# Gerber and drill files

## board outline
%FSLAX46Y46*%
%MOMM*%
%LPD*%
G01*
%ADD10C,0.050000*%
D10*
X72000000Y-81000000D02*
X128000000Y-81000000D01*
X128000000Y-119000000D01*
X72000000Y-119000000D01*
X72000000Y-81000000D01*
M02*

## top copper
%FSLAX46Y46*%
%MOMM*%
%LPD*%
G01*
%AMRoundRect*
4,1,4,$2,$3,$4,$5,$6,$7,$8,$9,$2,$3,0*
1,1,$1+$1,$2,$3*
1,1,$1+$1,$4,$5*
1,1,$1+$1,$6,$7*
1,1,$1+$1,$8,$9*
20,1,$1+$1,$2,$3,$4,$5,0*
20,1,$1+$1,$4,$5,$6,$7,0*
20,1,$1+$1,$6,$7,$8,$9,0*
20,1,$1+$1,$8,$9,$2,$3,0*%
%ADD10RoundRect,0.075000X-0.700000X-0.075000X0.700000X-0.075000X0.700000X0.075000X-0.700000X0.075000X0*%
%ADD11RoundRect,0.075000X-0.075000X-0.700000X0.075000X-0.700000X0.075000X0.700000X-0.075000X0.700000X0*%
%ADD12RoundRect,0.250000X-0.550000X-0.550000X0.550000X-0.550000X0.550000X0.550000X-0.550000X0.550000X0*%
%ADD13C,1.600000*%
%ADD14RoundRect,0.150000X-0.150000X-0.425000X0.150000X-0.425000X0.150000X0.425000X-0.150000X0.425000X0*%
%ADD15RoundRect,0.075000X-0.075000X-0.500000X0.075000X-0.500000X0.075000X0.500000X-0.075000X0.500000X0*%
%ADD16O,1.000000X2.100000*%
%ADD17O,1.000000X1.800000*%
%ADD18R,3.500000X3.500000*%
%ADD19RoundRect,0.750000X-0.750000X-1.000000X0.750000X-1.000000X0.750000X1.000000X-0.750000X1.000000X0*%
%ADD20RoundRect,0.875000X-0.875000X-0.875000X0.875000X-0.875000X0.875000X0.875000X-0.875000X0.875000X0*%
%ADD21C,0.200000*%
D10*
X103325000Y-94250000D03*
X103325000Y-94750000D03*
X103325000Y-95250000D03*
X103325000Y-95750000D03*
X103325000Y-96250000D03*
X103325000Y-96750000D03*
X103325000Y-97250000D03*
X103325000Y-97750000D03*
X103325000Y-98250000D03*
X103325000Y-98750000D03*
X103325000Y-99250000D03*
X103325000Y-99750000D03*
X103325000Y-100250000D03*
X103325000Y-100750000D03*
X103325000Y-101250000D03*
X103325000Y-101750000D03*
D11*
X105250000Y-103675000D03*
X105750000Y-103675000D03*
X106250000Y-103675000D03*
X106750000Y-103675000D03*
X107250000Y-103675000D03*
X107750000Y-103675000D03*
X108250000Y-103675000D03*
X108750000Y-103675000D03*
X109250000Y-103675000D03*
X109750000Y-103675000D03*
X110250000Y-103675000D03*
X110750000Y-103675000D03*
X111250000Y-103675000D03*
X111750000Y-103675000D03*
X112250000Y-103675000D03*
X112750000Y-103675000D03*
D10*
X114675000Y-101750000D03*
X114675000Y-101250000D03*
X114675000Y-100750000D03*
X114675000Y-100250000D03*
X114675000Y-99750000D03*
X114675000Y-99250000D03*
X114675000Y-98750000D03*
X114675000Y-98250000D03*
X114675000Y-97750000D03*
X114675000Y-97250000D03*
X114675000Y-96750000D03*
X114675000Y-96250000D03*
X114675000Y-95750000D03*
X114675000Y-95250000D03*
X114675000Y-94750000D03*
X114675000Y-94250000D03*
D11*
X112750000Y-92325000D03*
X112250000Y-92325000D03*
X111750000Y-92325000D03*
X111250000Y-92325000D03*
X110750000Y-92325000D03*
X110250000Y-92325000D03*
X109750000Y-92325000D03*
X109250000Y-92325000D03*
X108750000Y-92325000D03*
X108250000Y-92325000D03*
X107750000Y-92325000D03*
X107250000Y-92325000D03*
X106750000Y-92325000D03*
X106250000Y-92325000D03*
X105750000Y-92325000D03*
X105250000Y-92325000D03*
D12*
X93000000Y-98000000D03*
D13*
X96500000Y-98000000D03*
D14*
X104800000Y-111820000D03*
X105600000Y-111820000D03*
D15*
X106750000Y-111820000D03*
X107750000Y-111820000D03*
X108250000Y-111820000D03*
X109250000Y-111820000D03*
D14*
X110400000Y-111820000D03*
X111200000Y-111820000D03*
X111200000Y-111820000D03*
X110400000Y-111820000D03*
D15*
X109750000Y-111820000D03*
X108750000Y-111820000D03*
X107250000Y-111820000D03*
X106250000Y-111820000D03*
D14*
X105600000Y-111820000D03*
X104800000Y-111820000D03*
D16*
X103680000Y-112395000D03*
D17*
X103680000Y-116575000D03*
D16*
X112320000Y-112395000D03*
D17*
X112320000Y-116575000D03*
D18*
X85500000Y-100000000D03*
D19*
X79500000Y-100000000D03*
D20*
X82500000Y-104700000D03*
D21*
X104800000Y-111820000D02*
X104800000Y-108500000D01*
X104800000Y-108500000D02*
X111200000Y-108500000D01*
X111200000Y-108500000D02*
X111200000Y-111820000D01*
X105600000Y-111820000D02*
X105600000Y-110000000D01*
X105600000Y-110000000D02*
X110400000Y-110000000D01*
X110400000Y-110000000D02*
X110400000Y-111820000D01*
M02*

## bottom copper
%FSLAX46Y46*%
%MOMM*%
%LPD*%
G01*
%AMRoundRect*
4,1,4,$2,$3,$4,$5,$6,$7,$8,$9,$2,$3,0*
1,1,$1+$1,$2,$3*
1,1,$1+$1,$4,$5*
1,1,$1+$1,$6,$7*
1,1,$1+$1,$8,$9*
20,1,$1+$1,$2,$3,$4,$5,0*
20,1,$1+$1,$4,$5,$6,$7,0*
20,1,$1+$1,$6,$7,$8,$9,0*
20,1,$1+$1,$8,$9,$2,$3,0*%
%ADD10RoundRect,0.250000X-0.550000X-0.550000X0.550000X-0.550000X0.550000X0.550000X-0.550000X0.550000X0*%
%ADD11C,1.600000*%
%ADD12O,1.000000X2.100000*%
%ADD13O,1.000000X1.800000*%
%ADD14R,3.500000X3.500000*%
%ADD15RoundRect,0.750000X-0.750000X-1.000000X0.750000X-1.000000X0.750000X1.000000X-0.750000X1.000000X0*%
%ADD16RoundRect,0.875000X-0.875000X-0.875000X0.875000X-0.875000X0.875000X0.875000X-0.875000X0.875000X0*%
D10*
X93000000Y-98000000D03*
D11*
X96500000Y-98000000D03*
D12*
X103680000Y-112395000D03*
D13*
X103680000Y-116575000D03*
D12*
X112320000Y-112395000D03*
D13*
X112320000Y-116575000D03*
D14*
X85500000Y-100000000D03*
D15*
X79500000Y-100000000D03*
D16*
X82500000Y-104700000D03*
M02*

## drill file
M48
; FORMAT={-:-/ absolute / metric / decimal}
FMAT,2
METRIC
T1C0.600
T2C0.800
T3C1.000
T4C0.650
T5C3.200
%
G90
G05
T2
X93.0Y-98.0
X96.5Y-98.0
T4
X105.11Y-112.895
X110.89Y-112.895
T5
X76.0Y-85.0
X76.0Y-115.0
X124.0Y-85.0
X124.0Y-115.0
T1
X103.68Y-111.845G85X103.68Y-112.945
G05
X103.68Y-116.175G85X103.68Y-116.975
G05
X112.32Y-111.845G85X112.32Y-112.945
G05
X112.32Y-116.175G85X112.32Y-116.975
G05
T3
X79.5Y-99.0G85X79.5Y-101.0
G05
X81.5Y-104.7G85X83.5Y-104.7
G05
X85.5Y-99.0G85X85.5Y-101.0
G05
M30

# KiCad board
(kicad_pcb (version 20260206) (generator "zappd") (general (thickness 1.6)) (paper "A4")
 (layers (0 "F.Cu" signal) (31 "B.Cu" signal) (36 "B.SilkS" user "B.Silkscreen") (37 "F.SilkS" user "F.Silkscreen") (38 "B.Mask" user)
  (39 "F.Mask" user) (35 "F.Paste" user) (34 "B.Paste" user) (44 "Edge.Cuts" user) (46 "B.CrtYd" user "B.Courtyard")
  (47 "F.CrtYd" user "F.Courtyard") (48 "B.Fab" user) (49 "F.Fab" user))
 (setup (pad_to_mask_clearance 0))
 (gr_rect (start 72.0 81.0) (end 128.0 119.0) (stroke (width 0.05) (type default)) (fill none) (layer "Edge.Cuts"))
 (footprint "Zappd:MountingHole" (layer "F.Cu") (at 76.0 85.0)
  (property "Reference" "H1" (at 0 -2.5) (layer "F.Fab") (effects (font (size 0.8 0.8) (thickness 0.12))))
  (pad "" np_thru_hole circle (at 0 0) (size 3.2 3.2) (drill 3.2) (layers "*.Cu" "*.Mask")))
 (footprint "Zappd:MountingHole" (layer "F.Cu") (at 124.0 85.0)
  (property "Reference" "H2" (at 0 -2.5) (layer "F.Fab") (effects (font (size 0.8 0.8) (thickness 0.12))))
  (pad "" np_thru_hole circle (at 0 0) (size 3.2 3.2) (drill 3.2) (layers "*.Cu" "*.Mask")))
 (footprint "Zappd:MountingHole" (layer "F.Cu") (at 124.0 115.0)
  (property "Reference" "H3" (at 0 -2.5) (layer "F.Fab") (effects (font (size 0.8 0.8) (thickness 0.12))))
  (pad "" np_thru_hole circle (at 0 0) (size 3.2 3.2) (drill 3.2) (layers "*.Cu" "*.Mask")))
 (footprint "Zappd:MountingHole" (layer "F.Cu") (at 76.0 115.0)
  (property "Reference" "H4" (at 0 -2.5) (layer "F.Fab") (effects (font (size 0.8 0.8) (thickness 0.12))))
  (pad "" np_thru_hole circle (at 0 0) (size 3.2 3.2) (drill 3.2) (layers "*.Cu" "*.Mask")))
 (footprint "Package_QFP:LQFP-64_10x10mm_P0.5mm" (layer "F.Cu") (at 109 98)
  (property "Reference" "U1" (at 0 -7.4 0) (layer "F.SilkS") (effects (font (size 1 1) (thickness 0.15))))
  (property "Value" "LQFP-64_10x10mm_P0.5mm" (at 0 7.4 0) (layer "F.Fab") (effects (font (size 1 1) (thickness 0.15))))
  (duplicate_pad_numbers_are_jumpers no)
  (pad "1" smd roundrect (at -5.675 -3.75) (size 1.55 0.3) (layers "F.Cu" "F.Mask" "F.Paste") (roundrect_rratio 0.25))
  (pad "2" smd roundrect (at -5.675 -3.25) (size 1.55 0.3) (layers "F.Cu" "F.Mask" "F.Paste") (roundrect_rratio 0.25))
  (pad "3" smd roundrect (at -5.675 -2.75) (size 1.55 0.3) (layers "F.Cu" "F.Mask" "F.Paste") (roundrect_rratio 0.25))
  (pad "4" smd roundrect (at -5.675 -2.25) (size 1.55 0.3) (layers "F.Cu" "F.Mask" "F.Paste") (roundrect_rratio 0.25))
  (pad "5" smd roundrect (at -5.675 -1.75) (size 1.55 0.3) (layers "F.Cu" "F.Mask" "F.Paste") (roundrect_rratio 0.25))
  (pad "6" smd roundrect (at -5.675 -1.25) (size 1.55 0.3) (layers "F.Cu" "F.Mask" "F.Paste") (roundrect_rratio 0.25))
  (pad "7" smd roundrect (at -5.675 -0.75) (size 1.55 0.3) (layers "F.Cu" "F.Mask" "F.Paste") (roundrect_rratio 0.25))
  (pad "8" smd roundrect (at -5.675 -0.25) (size 1.55 0.3) (layers "F.Cu" "F.Mask" "F.Paste") (roundrect_rratio 0.25))
  (pad "9" smd roundrect (at -5.675 0.25) (size 1.55 0.3) (layers "F.Cu" "F.Mask" "F.Paste") (roundrect_rratio 0.25))
  (pad "10" smd roundrect (at -5.675 0.75) (size 1.55 0.3) (layers "F.Cu" "F.Mask" "F.Paste") (roundrect_rratio 0.25))
  (pad "11" smd roundrect (at -5.675 1.25) (size 1.55 0.3) (layers "F.Cu" "F.Mask" "F.Paste") (roundrect_rratio 0.25))
  (pad "12" smd roundrect (at -5.675 1.75) (size 1.55 0.3) (layers "F.Cu" "F.Mask" "F.Paste") (roundrect_rratio 0.25))
  (pad "13" smd roundrect (at -5.675 2.25) (size 1.55 0.3) (layers "F.Cu" "F.Mask" "F.Paste") (roundrect_rratio 0.25))
  (pad "14" smd roundrect (at -5.675 2.75) (size 1.55 0.3) (layers "F.Cu" "F.Mask" "F.Paste") (roundrect_rratio 0.25))
  (pad "15" smd roundrect (at -5.675 3.25) (size 1.55 0.3) (layers "F.Cu" "F.Mask" "F.Paste") (roundrect_rratio 0.25))
  (pad "16" smd roundrect (at -5.675 3.75) (size 1.55 0.3) (layers "F.Cu" "F.Mask" "F.Paste") (roundrect_rratio 0.25))
  (pad "17" smd roundrect (at -3.75 5.675) (size 0.3 1.55) (layers "F.Cu" "F.Mask" "F.Paste") (roundrect_rratio 0.25))
  (pad "18" smd roundrect (at -3.25 5.675) (size 0.3 1.55) (layers "F.Cu" "F.Mask" "F.Paste") (roundrect_rratio 0.25))
  (pad "19" smd roundrect (at -2.75 5.675) (size 0.3 1.55) (layers "F.Cu" "F.Mask" "F.Paste") (roundrect_rratio 0.25))
  (pad "20" smd roundrect (at -2.25 5.675) (size 0.3 1.55) (layers "F.Cu" "F.Mask" "F.Paste") (roundrect_rratio 0.25))
  (pad "21" smd roundrect (at -1.75 5.675) (size 0.3 1.55) (layers "F.Cu" "F.Mask" "F.Paste") (roundrect_rratio 0.25))
  (pad "22" smd roundrect (at -1.25 5.675) (size 0.3 1.55) (layers "F.Cu" "F.Mask" "F.Paste") (roundrect_rratio 0.25))
  (pad "23" smd roundrect (at -0.75 5.675) (size 0.3 1.55) (layers "F.Cu" "F.Mask" "F.Paste") (roundrect_rratio 0.25))
  (pad "24" smd roundrect (at -0.25 5.675) (size 0.3 1.55) (layers "F.Cu" "F.Mask" "F.Paste") (roundrect_rratio 0.25))
  (pad "25" smd roundrect (at 0.25 5.675) (size 0.3 1.55) (layers "F.Cu" "F.Mask" "F.Paste") (roundrect_rratio 0.25))
  (pad "26" smd roundrect (at 0.75 5.675) (size 0.3 1.55) (layers "F.Cu" "F.Mask" "F.Paste") (roundrect_rratio 0.25))
  (pad "27" smd roundrect (at 1.25 5.675) (size 0.3 1.55) (layers "F.Cu" "F.Mask" "F.Paste") (roundrect_rratio 0.25))
  (pad "28" smd roundrect (at 1.75 5.675) (size 0.3 1.55) (layers "F.Cu" "F.Mask" "F.Paste") (roundrect_rratio 0.25))
  (pad "29" smd roundrect (at 2.25 5.675) (size 0.3 1.55) (layers "F.Cu" "F.Mask" "F.Paste") (roundrect_rratio 0.25))
  (pad "30" smd roundrect (at 2.75 5.675) (size 0.3 1.55) (layers "F.Cu" "F.Mask" "F.Paste") (roundrect_rratio 0.25))
  (pad "31" smd roundrect (at 3.25 5.675) (size 0.3 1.55) (layers "F.Cu" "F.Mask" "F.Paste") (roundrect_rratio 0.25))
  (pad "32" smd roundrect (at 3.75 5.675) (size 0.3 1.55) (layers "F.Cu" "F.Mask" "F.Paste") (roundrect_rratio 0.25))
  (pad "33" smd roundrect (at 5.675 3.75) (size 1.55 0.3) (layers "F.Cu" "F.Mask" "F.Paste") (roundrect_rratio 0.25))
  (pad "34" smd roundrect (at 5.675 3.25) (size 1.55 0.3) (layers "F.Cu" "F.Mask" "F.Paste") (roundrect_rratio 0.25))
  (pad "35" smd roundrect (at 5.675 2.75) (size 1.55 0.3) (layers "F.Cu" "F.Mask" "F.Paste") (roundrect_rratio 0.25))
  (pad "36" smd roundrect (at 5.675 2.25) (size 1.55 0.3) (layers "F.Cu" "F.Mask" "F.Paste") (roundrect_rratio 0.25))
  (pad "37" smd roundrect (at 5.675 1.75) (size 1.55 0.3) (layers "F.Cu" "F.Mask" "F.Paste") (roundrect_rratio 0.25))
  (pad "38" smd roundrect (at 5.675 1.25) (size 1.55 0.3) (layers "F.Cu" "F.Mask" "F.Paste") (roundrect_rratio 0.25))
  (pad "39" smd roundrect (at 5.675 0.75) (size 1.55 0.3) (layers "F.Cu" "F.Mask" "F.Paste") (roundrect_rratio 0.25))
  (pad "40" smd roundrect (at 5.675 0.25) (size 1.55 0.3) (layers "F.Cu" "F.Mask" "F.Paste") (roundrect_rratio 0.25))
  (pad "41" smd roundrect (at 5.675 -0.25) (size 1.55 0.3) (layers "F.Cu" "F.Mask" "F.Paste") (roundrect_rratio 0.25))
  (pad "42" smd roundrect (at 5.675 -0.75) (size 1.55 0.3) (layers "F.Cu" "F.Mask" "F.Paste") (roundrect_rratio 0.25))
  (pad "43" smd roundrect (at 5.675 -1.25) (size 1.55 0.3) (layers "F.Cu" "F.Mask" "F.Paste") (roundrect_rratio 0.25))
  (pad "44" smd roundrect (at 5.675 -1.75) (size 1.55 0.3) (layers "F.Cu" "F.Mask" "F.Paste") (roundrect_rratio 0.25))
  (pad "45" smd roundrect (at 5.675 -2.25) (size 1.55 0.3) (layers "F.Cu" "F.Mask" "F.Paste") (roundrect_rratio 0.25))
  (pad "46" smd roundrect (at 5.675 -2.75) (size 1.55 0.3) (layers "F.Cu" "F.Mask" "F.Paste") (roundrect_rratio 0.25))
  (pad "47" smd roundrect (at 5.675 -3.25) (size 1.55 0.3) (layers "F.Cu" "F.Mask" "F.Paste") (roundrect_rratio 0.25))
  (pad "48" smd roundrect (at 5.675 -3.75) (size 1.55 0.3) (layers "F.Cu" "F.Mask" "F.Paste") (roundrect_rratio 0.25))
  (pad "49" smd roundrect (at 3.75 -5.675) (size 0.3 1.55) (layers "F.Cu" "F.Mask" "F.Paste") (roundrect_rratio 0.25))
  (pad "50" smd roundrect (at 3.25 -5.675) (size 0.3 1.55) (layers "F.Cu" "F.Mask" "F.Paste") (roundrect_rratio 0.25))
  (pad "51" smd roundrect (at 2.75 -5.675) (size 0.3 1.55) (layers "F.Cu" "F.Mask" "F.Paste") (roundrect_rratio 0.25))
  (pad "52" smd roundrect (at 2.25 -5.675) (size 0.3 1.55) (layers "F.Cu" "F.Mask" "F.Paste") (roundrect_rratio 0.25))
  (pad "53" smd roundrect (at 1.75 -5.675) (size 0.3 1.55) (layers "F.Cu" "F.Mask" "F.Paste") (roundrect_rratio 0.25))
  (pad "54" smd roundrect (at 1.25 -5.675) (size 0.3 1.55) (layers "F.Cu" "F.Mask" "F.Paste") (roundrect_rratio 0.25))
  (pad "55" smd roundrect (at 0.75 -5.675) (size 0.3 1.55) (layers "F.Cu" "F.Mask" "F.Paste") (roundrect_rratio 0.25))
  (pad "56" smd roundrect (at 0.25 -5.675) (size 0.3 1.55) (layers "F.Cu" "F.Mask" "F.Paste") (roundrect_rratio 0.25))
  (pad "57" smd roundrect (at -0.25 -5.675) (size 0.3 1.55) (layers "F.Cu" "F.Mask" "F.Paste") (roundrect_rratio 0.25))
  (pad "58" smd roundrect (at -0.75 -5.675) (size 0.3 1.55) (layers "F.Cu" "F.Mask" "F.Paste") (roundrect_rratio 0.25))
  (pad "59" smd roundrect (at -1.25 -5.675) (size 0.3 1.55) (layers "F.Cu" "F.Mask" "F.Paste") (roundrect_rratio 0.25))
  (pad "60" smd roundrect (at -1.75 -5.675) (size 0.3 1.55) (layers "F.Cu" "F.Mask" "F.Paste") (roundrect_rratio 0.25))
  (pad "61" smd roundrect (at -2.25 -5.675) (size 0.3 1.55) (layers "F.Cu" "F.Mask" "F.Paste") (roundrect_rratio 0.25))
  (pad "62" smd roundrect (at -2.75 -5.675) (size 0.3 1.55) (layers "F.Cu" "F.Mask" "F.Paste") (roundrect_rratio 0.25))
  (pad "63" smd roundrect (at -3.25 -5.675) (size 0.3 1.55) (layers "F.Cu" "F.Mask" "F.Paste") (roundrect_rratio 0.25))
  (pad "64" smd roundrect (at -3.75 -5.675) (size 0.3 1.55) (layers "F.Cu" "F.Mask" "F.Paste") (roundrect_rratio 0.25)))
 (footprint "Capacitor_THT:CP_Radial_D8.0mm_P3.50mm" (layer "F.Cu") (at 93 98)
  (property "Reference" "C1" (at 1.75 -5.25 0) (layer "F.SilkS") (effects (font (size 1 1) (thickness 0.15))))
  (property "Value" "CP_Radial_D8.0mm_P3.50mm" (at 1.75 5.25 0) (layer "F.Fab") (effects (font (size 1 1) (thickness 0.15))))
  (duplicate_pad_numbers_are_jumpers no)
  (pad "1" thru_hole roundrect (at 0 0) (size 1.6 1.6) (drill 0.8) (layers "*.Cu" "*.Mask") (remove_unused_layers no)
   (roundrect_rratio 0.15625))
  (pad "2" thru_hole circle (at 3.5 0) (size 1.6 1.6) (drill 0.8) (layers "*.Cu" "*.Mask") (remove_unused_layers no)))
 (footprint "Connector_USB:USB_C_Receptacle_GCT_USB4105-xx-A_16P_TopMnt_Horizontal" (layer "F.Cu") (at 108 115.5)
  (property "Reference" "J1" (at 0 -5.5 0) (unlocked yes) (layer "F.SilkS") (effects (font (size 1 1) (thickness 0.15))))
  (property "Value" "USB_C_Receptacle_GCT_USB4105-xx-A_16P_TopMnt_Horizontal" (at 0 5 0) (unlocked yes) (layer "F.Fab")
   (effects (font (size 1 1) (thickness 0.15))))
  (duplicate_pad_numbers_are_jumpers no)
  (pad "" np_thru_hole circle (at -2.89 -2.605) (size 0.65 0.65) (drill 0.65) (layers "*.Cu" "*.Mask"))
  (pad "" np_thru_hole circle (at 2.89 -2.605) (size 0.65 0.65) (drill 0.65) (layers "*.Cu" "*.Mask"))
  (pad "A1" smd roundrect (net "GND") (at -3.2 -3.68) (size 0.6 1.15) (layers "F.Cu" "F.Mask" "F.Paste") (roundrect_rratio 0.25))
  (pad "A4" smd roundrect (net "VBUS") (at -2.4 -3.68) (size 0.6 1.15) (layers "F.Cu" "F.Mask" "F.Paste") (roundrect_rratio 0.25))
  (pad "A5" smd roundrect (at -1.25 -3.68) (size 0.3 1.15) (layers "F.Cu" "F.Mask" "F.Paste") (roundrect_rratio 0.25))
  (pad "A6" smd roundrect (at -0.25 -3.68) (size 0.3 1.15) (layers "F.Cu" "F.Mask" "F.Paste") (roundrect_rratio 0.25))
  (pad "A7" smd roundrect (at 0.25 -3.68) (size 0.3 1.15) (layers "F.Cu" "F.Mask" "F.Paste") (roundrect_rratio 0.25))
  (pad "A8" smd roundrect (at 1.25 -3.68) (size 0.3 1.15) (layers "F.Cu" "F.Mask" "F.Paste") (roundrect_rratio 0.25))
  (pad "A9" smd roundrect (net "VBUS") (at 2.4 -3.68) (size 0.6 1.15) (layers "F.Cu" "F.Mask" "F.Paste") (roundrect_rratio 0.25))
  (pad "A12" smd roundrect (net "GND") (at 3.2 -3.68) (size 0.6 1.15) (layers "F.Cu" "F.Mask" "F.Paste") (roundrect_rratio 0.25))
  (pad "B1" smd roundrect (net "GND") (at 3.2 -3.68) (size 0.6 1.15) (layers "F.Cu" "F.Mask" "F.Paste") (roundrect_rratio 0.25))
  (pad "B4" smd roundrect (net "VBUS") (at 2.4 -3.68) (size 0.6 1.15) (layers "F.Cu" "F.Mask" "F.Paste") (roundrect_rratio 0.25))
  (pad "B5" smd roundrect (at 1.75 -3.68) (size 0.3 1.15) (layers "F.Cu" "F.Mask" "F.Paste") (roundrect_rratio 0.25))
  (pad "B6" smd roundrect (at 0.75 -3.68) (size 0.3 1.15) (layers "F.Cu" "F.Mask" "F.Paste") (roundrect_rratio 0.25))
  (pad "B7" smd roundrect (at -0.75 -3.68) (size 0.3 1.15) (layers "F.Cu" "F.Mask" "F.Paste") (roundrect_rratio 0.25))
  (pad "B8" smd roundrect (at -1.75 -3.68) (size 0.3 1.15) (layers "F.Cu" "F.Mask" "F.Paste") (roundrect_rratio 0.25))
  (pad "B9" smd roundrect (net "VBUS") (at -2.4 -3.68) (size 0.6 1.15) (layers "F.Cu" "F.Mask" "F.Paste") (roundrect_rratio 0.25))
  (pad "B12" smd roundrect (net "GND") (at -3.2 -3.68) (size 0.6 1.15) (layers "F.Cu" "F.Mask" "F.Paste") (roundrect_rratio 0.25))
  (pad "SH" thru_hole oval (at -4.32 -3.105) (size 1 2.1) (drill oval 0.6 1.7) (layers "*.Cu" "*.Mask" "F.Paste") (remove_unused_layers no))
  (pad "SH" thru_hole oval (at -4.32 1.075) (size 1 1.8) (drill oval 0.6 1.4) (layers "*.Cu" "*.Mask" "F.Paste") (remove_unused_layers no))
  (pad "SH" thru_hole oval (at 4.32 -3.105) (size 1 2.1) (drill oval 0.6 1.7) (layers "*.Cu" "*.Mask" "F.Paste") (remove_unused_layers no))
  (pad "SH" thru_hole oval (at 4.32 1.075) (size 1 1.8) (drill oval 0.6 1.4) (layers "*.Cu" "*.Mask" "F.Paste") (remove_unused_layers no)))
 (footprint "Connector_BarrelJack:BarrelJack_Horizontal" (layer "F.Cu") (at 85.5 100)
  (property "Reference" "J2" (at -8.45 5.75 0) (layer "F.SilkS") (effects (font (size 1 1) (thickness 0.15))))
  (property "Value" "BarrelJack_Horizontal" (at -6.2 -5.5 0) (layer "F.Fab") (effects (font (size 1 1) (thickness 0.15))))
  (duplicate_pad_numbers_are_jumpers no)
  (pad "1" thru_hole rect (at 0 0) (size 3.5 3.5) (drill oval 1 3) (layers "*.Cu" "*.Mask") (remove_unused_layers no))
  (pad "2" thru_hole roundrect (at -6 0) (size 3 3.5) (drill oval 1 3) (layers "*.Cu" "*.Mask") (remove_unused_layers no)
   (roundrect_rratio 0.25))
  (pad "3" thru_hole roundrect (at -3 4.7) (size 3.5 3.5) (drill oval 3 1) (layers "*.Cu" "*.Mask") (remove_unused_layers no)
   (roundrect_rratio 0.25)))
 (segment (start 104.8000 111.8200) (end 104.8000 108.5000) (width 0.2) (layer "F.Cu") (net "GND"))
 (segment (start 104.8000 108.5000) (end 111.2000 108.5000) (width 0.2) (layer "F.Cu") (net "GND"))
 (segment (start 111.2000 108.5000) (end 111.2000 111.8200) (width 0.2) (layer "F.Cu") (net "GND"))
 (segment (start 105.6000 111.8200) (end 105.6000 110.0000) (width 0.2) (layer "F.Cu") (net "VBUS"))
 (segment (start 105.6000 110.0000) (end 110.4000 110.0000) (width 0.2) (layer "F.Cu") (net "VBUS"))
 (segment (start 110.4000 110.0000) (end 110.4000 111.8200) (width 0.2) (layer "F.Cu") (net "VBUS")))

